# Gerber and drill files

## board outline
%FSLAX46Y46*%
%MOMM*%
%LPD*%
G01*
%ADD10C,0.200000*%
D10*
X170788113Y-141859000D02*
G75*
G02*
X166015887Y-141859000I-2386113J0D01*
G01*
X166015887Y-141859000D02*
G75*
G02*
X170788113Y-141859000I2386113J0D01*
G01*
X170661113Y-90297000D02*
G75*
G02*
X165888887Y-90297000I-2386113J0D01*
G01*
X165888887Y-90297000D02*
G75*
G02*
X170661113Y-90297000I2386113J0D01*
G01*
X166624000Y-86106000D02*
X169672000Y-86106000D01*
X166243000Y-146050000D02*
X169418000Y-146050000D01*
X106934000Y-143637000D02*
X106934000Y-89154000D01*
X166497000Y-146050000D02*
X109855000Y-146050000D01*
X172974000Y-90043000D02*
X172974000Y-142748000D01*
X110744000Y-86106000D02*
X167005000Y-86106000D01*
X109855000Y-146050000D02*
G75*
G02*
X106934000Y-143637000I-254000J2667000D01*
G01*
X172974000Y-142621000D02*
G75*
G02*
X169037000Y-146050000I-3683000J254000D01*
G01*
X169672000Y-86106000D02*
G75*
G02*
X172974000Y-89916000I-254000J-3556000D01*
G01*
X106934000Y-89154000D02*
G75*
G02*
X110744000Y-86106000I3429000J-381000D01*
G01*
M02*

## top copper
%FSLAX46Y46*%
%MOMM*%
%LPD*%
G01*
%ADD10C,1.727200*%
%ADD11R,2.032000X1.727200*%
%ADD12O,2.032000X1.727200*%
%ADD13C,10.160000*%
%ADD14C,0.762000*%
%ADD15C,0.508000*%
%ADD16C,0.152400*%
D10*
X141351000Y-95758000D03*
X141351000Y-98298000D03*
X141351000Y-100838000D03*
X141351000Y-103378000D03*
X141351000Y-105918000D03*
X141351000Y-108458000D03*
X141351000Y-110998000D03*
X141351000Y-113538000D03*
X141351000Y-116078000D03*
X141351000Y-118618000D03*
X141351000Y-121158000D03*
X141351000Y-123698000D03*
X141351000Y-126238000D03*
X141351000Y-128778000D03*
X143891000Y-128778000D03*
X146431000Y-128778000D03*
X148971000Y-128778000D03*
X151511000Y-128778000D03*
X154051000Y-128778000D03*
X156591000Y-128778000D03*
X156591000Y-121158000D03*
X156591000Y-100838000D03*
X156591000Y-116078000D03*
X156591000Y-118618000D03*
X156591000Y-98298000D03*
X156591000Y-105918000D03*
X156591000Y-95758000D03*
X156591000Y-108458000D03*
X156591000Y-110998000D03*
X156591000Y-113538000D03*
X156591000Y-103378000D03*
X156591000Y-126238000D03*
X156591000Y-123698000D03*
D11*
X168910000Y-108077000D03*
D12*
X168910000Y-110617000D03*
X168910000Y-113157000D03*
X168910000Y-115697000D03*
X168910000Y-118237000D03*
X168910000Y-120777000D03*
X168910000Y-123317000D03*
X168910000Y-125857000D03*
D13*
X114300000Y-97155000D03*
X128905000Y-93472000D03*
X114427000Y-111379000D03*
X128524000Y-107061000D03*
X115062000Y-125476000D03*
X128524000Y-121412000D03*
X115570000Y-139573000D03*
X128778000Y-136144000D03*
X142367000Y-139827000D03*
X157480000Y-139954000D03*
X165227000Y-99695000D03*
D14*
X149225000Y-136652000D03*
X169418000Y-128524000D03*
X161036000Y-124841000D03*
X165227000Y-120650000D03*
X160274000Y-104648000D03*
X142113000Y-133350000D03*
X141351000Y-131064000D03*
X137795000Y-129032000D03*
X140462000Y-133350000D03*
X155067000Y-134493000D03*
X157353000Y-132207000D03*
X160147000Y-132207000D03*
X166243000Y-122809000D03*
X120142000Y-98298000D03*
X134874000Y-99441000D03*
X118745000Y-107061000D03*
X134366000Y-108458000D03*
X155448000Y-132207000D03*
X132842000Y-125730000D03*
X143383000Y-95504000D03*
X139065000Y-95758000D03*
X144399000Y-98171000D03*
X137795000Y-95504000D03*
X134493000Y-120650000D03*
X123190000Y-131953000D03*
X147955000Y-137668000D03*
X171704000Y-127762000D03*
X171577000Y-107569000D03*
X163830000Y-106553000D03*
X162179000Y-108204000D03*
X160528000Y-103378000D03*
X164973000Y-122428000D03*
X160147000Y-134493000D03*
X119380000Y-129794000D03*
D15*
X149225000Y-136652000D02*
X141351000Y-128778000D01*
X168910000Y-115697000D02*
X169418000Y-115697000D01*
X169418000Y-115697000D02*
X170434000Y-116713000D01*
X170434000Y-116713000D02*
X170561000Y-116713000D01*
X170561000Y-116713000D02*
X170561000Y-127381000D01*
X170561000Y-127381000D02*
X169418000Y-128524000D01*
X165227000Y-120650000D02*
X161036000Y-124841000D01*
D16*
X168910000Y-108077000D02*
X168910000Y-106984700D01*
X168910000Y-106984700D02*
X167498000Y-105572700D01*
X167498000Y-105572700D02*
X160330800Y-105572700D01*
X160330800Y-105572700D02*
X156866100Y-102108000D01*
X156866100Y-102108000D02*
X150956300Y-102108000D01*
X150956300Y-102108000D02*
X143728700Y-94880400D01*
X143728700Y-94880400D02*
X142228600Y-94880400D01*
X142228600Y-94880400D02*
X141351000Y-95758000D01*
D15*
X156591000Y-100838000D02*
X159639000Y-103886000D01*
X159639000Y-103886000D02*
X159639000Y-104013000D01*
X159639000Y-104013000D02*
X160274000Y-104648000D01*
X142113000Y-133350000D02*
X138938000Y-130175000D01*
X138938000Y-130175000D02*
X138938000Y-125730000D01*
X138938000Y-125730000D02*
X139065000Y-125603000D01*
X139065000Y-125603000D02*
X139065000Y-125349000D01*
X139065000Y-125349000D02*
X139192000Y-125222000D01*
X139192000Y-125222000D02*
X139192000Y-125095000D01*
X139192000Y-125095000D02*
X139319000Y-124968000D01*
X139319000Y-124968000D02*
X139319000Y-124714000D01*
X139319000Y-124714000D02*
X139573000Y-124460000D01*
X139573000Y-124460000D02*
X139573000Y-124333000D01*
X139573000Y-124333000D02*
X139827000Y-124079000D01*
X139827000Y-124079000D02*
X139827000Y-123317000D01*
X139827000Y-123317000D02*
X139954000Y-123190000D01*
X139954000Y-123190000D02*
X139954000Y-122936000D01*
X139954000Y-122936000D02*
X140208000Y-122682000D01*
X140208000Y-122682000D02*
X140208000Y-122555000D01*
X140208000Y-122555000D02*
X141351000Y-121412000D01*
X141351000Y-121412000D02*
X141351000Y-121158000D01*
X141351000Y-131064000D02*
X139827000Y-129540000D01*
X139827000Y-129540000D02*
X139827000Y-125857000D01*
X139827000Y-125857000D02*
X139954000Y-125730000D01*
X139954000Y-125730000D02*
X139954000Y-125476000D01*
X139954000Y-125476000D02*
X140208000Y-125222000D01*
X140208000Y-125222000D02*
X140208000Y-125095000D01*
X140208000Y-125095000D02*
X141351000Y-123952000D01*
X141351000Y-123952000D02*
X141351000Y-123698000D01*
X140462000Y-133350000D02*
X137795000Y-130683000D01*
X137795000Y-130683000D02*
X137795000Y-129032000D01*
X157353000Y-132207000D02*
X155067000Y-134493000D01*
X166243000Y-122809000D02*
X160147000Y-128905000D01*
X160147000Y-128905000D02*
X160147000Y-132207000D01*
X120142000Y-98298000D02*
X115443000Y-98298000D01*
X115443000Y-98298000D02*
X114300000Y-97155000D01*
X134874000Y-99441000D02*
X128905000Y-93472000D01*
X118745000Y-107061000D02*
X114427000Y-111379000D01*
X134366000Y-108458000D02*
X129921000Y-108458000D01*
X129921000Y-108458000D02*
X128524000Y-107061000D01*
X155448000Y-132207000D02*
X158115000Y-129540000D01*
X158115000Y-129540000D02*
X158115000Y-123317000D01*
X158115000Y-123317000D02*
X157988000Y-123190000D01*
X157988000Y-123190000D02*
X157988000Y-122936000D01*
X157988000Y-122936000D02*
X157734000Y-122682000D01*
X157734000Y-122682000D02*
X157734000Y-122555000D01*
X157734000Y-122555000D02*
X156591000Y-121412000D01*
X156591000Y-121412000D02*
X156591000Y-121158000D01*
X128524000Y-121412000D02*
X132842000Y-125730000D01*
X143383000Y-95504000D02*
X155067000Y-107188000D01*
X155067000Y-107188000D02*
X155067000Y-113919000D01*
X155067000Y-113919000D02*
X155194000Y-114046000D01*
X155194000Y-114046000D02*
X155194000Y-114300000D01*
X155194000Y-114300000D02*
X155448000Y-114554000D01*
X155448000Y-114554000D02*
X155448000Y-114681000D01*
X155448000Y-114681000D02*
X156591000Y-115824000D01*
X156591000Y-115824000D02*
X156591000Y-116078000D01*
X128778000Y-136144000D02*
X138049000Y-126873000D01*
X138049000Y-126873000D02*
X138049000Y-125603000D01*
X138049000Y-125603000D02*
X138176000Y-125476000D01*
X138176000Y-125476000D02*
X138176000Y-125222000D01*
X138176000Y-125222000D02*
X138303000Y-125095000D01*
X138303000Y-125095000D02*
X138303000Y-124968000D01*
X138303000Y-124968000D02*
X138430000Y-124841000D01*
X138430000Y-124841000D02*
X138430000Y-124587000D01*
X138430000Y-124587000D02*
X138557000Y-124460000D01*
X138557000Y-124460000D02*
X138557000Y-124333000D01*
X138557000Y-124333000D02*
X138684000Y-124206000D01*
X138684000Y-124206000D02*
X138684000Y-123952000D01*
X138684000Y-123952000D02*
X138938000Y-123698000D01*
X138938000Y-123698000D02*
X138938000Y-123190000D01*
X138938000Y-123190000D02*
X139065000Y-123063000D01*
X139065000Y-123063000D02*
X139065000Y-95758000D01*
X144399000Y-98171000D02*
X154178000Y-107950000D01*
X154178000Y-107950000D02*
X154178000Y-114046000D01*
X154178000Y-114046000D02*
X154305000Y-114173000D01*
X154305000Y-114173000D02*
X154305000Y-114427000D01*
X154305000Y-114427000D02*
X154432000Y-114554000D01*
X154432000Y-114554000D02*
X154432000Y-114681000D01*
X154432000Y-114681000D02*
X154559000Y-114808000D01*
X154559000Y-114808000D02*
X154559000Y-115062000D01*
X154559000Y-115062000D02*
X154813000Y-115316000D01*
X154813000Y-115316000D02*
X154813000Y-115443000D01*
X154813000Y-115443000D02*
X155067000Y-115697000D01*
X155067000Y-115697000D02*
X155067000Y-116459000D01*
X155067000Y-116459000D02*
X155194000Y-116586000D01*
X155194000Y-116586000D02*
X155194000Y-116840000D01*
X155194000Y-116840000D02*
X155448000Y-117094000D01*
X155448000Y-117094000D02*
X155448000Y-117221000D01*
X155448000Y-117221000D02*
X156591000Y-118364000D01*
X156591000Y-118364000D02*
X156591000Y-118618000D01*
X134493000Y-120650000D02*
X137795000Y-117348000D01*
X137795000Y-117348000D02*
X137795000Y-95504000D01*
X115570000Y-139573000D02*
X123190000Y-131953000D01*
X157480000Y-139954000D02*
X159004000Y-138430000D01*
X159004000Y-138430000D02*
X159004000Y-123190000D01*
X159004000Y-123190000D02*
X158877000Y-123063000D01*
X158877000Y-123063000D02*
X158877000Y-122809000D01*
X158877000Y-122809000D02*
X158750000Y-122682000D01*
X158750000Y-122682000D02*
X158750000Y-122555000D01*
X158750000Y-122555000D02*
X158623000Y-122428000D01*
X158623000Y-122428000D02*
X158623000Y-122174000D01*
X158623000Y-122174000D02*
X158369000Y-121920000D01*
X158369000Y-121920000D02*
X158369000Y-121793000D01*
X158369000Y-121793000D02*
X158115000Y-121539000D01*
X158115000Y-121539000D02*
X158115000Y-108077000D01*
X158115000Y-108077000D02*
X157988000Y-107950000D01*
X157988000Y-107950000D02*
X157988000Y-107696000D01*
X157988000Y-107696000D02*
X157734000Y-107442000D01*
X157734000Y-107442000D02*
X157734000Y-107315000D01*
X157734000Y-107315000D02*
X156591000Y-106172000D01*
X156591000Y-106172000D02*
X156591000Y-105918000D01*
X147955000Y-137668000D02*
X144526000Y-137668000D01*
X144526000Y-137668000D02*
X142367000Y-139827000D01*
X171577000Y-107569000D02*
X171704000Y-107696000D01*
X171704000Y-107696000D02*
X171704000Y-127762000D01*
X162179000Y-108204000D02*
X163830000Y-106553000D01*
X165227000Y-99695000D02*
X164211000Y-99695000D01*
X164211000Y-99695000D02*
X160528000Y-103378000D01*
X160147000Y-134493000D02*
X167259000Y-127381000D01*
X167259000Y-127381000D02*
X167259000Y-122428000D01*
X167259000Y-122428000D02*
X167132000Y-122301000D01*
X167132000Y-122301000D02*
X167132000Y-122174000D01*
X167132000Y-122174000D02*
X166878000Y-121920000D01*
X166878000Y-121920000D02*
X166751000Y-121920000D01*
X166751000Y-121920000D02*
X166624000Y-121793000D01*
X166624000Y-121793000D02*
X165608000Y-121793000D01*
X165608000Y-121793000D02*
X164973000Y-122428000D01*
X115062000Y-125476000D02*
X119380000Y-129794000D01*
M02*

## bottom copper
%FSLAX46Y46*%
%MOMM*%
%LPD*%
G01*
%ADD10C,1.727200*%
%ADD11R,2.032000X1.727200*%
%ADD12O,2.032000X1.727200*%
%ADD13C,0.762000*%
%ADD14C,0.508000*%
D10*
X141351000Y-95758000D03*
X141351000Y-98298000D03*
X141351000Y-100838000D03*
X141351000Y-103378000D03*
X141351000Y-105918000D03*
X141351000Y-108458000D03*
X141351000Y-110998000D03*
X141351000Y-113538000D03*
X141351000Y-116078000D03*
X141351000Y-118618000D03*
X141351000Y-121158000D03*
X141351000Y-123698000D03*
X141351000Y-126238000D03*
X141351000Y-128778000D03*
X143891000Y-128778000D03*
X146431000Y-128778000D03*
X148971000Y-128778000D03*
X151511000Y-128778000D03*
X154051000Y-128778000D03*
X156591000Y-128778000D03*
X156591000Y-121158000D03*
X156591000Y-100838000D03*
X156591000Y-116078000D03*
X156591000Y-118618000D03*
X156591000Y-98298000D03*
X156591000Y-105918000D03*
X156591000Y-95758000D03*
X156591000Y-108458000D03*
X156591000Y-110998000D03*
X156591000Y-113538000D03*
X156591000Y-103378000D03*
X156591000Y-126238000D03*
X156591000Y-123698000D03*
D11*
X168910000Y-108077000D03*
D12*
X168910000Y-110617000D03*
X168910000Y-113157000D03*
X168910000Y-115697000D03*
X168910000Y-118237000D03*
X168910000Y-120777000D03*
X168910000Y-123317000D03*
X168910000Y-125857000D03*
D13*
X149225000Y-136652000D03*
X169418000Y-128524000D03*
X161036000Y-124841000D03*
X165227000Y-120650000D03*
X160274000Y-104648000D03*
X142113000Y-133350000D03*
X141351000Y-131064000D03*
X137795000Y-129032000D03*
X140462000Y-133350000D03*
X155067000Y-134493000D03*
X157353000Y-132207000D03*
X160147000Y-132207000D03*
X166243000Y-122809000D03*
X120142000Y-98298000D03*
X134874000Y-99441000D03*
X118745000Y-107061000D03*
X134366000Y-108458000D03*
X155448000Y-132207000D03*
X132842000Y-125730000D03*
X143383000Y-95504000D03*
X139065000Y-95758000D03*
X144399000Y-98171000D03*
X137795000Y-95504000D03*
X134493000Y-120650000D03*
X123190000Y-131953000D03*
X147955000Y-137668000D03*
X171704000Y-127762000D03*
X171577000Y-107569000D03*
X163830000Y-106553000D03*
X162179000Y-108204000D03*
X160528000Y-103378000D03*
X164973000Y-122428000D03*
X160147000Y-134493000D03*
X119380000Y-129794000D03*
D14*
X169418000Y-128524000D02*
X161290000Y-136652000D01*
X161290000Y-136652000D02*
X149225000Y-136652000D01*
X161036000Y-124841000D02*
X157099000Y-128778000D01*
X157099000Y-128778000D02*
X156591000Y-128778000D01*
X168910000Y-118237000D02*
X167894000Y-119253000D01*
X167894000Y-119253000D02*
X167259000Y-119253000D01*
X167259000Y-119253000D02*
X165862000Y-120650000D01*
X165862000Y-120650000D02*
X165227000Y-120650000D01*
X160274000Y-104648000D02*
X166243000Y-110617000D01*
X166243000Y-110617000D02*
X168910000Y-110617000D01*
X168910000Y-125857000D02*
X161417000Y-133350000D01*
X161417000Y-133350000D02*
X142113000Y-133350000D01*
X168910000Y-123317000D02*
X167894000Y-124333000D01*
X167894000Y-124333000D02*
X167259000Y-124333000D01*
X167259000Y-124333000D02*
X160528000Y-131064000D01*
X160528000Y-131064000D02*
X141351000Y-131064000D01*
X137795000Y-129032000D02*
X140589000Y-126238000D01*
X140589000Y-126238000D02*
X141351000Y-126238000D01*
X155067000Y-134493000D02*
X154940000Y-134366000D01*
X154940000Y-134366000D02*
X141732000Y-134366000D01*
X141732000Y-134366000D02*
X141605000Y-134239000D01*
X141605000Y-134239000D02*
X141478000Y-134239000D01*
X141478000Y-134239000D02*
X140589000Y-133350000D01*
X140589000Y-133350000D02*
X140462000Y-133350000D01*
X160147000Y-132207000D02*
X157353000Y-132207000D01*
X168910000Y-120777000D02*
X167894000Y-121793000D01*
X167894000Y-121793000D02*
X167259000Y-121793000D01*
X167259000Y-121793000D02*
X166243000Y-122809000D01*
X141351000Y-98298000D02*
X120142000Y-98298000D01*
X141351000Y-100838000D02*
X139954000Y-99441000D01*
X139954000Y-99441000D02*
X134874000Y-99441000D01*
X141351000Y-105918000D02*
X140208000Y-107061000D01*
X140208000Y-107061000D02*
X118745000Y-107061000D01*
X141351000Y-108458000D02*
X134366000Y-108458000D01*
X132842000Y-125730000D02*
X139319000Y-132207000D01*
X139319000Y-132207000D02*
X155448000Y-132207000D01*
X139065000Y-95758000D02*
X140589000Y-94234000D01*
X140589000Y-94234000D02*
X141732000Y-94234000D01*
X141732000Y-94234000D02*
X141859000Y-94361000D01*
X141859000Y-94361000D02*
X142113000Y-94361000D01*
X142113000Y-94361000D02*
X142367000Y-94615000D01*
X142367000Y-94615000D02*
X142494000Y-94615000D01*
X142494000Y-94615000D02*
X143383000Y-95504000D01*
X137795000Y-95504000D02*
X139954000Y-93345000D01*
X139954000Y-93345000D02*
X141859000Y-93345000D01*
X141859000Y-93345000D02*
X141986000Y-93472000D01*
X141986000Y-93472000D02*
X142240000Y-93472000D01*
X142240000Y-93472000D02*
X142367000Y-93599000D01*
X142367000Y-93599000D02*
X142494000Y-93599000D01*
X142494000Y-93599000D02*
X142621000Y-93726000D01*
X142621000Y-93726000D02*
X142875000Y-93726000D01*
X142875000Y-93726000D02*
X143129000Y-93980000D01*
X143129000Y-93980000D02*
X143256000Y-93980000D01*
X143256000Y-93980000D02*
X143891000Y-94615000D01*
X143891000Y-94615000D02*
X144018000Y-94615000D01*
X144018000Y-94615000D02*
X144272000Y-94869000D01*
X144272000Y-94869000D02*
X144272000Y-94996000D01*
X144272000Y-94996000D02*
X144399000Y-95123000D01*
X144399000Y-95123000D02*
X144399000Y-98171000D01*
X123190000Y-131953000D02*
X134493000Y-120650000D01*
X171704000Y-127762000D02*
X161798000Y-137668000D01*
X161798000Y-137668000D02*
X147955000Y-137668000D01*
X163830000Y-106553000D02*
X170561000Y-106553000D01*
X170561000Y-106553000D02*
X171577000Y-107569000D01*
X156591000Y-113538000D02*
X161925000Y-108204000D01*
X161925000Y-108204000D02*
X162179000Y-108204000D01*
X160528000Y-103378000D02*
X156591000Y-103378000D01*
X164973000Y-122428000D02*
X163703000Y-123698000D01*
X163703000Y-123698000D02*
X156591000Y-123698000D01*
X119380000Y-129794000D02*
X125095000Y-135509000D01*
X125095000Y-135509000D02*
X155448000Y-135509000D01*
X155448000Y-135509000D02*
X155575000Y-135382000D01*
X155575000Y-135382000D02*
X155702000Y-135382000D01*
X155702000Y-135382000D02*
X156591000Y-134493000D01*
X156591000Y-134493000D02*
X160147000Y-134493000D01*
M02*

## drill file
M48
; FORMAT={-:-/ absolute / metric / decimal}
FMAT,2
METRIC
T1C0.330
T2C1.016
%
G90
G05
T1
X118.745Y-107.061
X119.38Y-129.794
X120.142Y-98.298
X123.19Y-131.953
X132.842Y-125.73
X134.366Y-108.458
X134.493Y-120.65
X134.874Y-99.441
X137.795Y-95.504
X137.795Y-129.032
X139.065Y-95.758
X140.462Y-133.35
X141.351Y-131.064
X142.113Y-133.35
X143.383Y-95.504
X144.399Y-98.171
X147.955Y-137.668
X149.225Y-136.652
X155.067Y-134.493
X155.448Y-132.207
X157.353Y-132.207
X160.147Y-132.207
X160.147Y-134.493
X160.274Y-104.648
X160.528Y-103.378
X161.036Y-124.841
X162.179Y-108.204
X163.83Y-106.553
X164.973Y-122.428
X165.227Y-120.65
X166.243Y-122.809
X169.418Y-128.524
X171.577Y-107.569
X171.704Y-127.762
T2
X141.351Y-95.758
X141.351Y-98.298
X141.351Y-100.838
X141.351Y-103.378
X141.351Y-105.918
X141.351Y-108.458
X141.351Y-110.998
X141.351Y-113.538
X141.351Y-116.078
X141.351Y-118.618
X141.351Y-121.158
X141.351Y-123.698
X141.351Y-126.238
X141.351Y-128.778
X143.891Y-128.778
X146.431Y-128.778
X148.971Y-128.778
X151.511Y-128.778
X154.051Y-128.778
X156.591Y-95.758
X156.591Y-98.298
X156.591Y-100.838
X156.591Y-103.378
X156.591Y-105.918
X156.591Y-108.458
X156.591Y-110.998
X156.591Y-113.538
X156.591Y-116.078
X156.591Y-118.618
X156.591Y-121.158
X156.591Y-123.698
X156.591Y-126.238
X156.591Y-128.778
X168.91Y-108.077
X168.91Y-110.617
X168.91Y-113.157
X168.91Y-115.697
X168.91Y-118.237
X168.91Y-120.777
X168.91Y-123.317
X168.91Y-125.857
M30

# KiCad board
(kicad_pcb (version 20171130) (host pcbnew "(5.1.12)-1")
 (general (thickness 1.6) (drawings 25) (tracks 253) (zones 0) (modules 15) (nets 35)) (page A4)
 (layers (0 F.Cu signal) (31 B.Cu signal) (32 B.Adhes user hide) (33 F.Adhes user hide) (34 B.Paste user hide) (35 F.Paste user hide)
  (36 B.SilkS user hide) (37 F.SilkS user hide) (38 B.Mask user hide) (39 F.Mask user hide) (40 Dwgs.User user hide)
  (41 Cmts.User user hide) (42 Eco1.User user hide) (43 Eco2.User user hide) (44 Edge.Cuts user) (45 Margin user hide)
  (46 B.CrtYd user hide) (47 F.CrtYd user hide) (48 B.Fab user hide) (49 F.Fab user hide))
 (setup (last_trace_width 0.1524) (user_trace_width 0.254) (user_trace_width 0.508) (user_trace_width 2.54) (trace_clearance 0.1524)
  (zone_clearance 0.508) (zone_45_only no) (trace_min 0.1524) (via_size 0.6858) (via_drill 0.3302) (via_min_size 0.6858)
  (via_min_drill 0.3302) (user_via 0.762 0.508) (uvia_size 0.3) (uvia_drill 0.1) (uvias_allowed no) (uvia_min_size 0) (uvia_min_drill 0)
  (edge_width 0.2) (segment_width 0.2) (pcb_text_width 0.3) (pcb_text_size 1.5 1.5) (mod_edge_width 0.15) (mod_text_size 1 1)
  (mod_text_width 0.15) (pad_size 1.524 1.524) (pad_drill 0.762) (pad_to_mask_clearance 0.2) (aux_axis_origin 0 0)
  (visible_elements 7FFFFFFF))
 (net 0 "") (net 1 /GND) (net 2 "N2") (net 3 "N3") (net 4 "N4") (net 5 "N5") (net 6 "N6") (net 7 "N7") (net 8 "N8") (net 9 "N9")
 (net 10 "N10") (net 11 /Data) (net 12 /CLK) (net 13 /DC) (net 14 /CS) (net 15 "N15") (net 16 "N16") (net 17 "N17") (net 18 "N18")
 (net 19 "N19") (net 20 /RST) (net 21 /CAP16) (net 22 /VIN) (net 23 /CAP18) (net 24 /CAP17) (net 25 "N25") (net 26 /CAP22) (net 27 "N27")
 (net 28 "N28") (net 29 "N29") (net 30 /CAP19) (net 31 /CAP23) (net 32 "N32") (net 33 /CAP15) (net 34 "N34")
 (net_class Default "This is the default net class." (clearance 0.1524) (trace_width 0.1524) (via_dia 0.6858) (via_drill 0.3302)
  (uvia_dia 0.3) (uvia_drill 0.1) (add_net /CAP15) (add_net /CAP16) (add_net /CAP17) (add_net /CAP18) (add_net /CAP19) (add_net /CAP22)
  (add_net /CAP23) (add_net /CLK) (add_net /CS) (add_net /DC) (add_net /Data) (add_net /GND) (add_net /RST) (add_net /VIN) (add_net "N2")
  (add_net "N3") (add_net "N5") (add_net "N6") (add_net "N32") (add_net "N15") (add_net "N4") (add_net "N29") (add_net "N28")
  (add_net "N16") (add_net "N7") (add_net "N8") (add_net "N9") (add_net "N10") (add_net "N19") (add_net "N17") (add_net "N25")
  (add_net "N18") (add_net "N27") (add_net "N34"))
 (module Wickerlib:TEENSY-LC (layer F.Cu) (at 151.511 105.918)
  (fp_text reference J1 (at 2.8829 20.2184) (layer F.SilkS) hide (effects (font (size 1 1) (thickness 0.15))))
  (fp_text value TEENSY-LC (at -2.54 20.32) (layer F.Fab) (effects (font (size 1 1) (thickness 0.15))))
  (pad G1 thru_hole circle (at -10.16 -10.16) (size 1.7272 1.7272) (drill 1.016) (layers *.Cu *.Mask F.SilkS) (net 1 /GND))
  (pad 0 thru_hole circle (at -10.16 -7.62) (size 1.7272 1.7272) (drill 1.016) (layers *.Cu *.Mask F.SilkS) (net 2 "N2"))
  (pad 1 thru_hole circle (at -10.16 -5.08) (size 1.7272 1.7272) (drill 1.016) (layers *.Cu *.Mask F.SilkS) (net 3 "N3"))
  (pad 2 thru_hole circle (at -10.16 -2.54) (size 1.7272 1.7272) (drill 1.016) (layers *.Cu *.Mask F.SilkS) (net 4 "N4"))
  (pad 3 thru_hole circle (at -10.16 0) (size 1.7272 1.7272) (drill 1.016) (layers *.Cu *.Mask F.SilkS) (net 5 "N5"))
  (pad 4 thru_hole circle (at -10.16 2.54) (size 1.7272 1.7272) (drill 1.016) (layers *.Cu *.Mask F.SilkS) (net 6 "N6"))
  (pad 5 thru_hole circle (at -10.16 5.08) (size 1.7272 1.7272) (drill 1.016) (layers *.Cu *.Mask F.SilkS) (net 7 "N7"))
  (pad 6 thru_hole circle (at -10.16 7.62) (size 1.7272 1.7272) (drill 1.016) (layers *.Cu *.Mask F.SilkS) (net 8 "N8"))
  (pad 7 thru_hole circle (at -10.16 10.16) (size 1.7272 1.7272) (drill 1.016) (layers *.Cu *.Mask F.SilkS) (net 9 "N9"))
  (pad 8 thru_hole circle (at -10.16 12.7) (size 1.7272 1.7272) (drill 1.016) (layers *.Cu *.Mask F.SilkS) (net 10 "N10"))
  (pad 9 thru_hole circle (at -10.16 15.24) (size 1.7272 1.7272) (drill 1.016) (layers *.Cu *.Mask F.SilkS) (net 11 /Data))
  (pad 10 thru_hole circle (at -10.16 17.78) (size 1.7272 1.7272) (drill 1.016) (layers *.Cu *.Mask F.SilkS) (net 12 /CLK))
  (pad 11 thru_hole circle (at -10.16 20.32) (size 1.7272 1.7272) (drill 1.016) (layers *.Cu *.Mask F.SilkS) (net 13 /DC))
  (pad 12 thru_hole circle (at -10.16 22.86) (size 1.7272 1.7272) (drill 1.016) (layers *.Cu *.Mask F.SilkS) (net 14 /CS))
  (pad 17A thru_hole circle (at -7.62 22.86) (size 1.7272 1.7272) (drill 1.016) (layers *.Cu *.Mask F.SilkS) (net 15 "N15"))
  (pad 3V1 thru_hole circle (at -5.08 22.86) (size 1.7272 1.7272) (drill 1.016) (layers *.Cu *.Mask F.SilkS) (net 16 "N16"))
  (pad G2 thru_hole circle (at -2.54 22.86) (size 1.7272 1.7272) (drill 1.016) (layers *.Cu *.Mask F.SilkS) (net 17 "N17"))
  (pad PGM thru_hole circle (at 0 22.86) (size 1.7272 1.7272) (drill 1.016) (layers *.Cu *.Mask F.SilkS) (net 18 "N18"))
  (pad DAC thru_hole circle (at 2.54 22.86) (size 1.7272 1.7272) (drill 1.016) (layers *.Cu *.Mask F.SilkS) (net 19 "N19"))
  (pad 13 thru_hole circle (at 5.08 22.86) (size 1.7272 1.7272) (drill 1.016) (layers *.Cu *.Mask F.SilkS) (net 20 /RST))
  (pad 16 thru_hole circle (at 5.08 15.24) (size 1.7272 1.7272) (drill 1.016) (layers *.Cu *.Mask F.SilkS) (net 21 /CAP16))
  (pad 3V2 thru_hole circle (at 5.08 -5.08) (size 1.7272 1.7272) (drill 1.016) (layers *.Cu *.Mask F.SilkS) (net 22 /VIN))
  (pad 18 thru_hole circle (at 5.08 10.16) (size 1.7272 1.7272) (drill 1.016) (layers *.Cu *.Mask F.SilkS) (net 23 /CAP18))
  (pad 17 thru_hole circle (at 5.08 12.7) (size 1.7272 1.7272) (drill 1.016) (layers *.Cu *.Mask F.SilkS) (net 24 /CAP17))
  (pad G3 thru_hole circle (at 5.08 -7.62) (size 1.7272 1.7272) (drill 1.016) (layers *.Cu *.Mask F.SilkS) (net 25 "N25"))
  (pad 22 thru_hole circle (at 5.08 0) (size 1.7272 1.7272) (drill 1.016) (layers *.Cu *.Mask F.SilkS) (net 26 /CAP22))
  (pad VIN thru_hole circle (at 5.08 -10.16) (size 1.7272 1.7272) (drill 1.016) (layers *.Cu *.Mask F.SilkS) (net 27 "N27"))
  (pad 21 thru_hole circle (at 5.08 2.54) (size 1.7272 1.7272) (drill 1.016) (layers *.Cu *.Mask F.SilkS) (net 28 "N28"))
  (pad 20 thru_hole circle (at 5.08 5.08) (size 1.7272 1.7272) (drill 1.016) (layers *.Cu *.Mask F.SilkS) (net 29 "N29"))
  (pad 19 thru_hole circle (at 5.08 7.62) (size 1.7272 1.7272) (drill 1.016) (layers *.Cu *.Mask F.SilkS) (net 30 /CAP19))
  (pad 23 thru_hole circle (at 5.08 -2.54) (size 1.7272 1.7272) (drill 1.016) (layers *.Cu *.Mask F.SilkS) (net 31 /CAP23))
  (pad 14 thru_hole circle (at 5.08 20.32) (size 1.7272 1.7272) (drill 1.016) (layers *.Cu *.Mask F.SilkS) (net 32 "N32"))
  (pad 15 thru_hole circle (at 5.08 17.78) (size 1.7272 1.7272) (drill 1.016) (layers *.Cu *.Mask F.SilkS) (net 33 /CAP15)))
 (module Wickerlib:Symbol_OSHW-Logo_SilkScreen (layer F.Cu) (at 167.767 133.985 270)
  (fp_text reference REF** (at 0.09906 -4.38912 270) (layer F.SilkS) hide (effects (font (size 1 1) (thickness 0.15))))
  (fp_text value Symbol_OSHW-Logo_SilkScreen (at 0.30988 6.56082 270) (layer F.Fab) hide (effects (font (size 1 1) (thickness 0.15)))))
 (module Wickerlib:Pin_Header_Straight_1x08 (layer F.Cu) (at 168.91 108.077)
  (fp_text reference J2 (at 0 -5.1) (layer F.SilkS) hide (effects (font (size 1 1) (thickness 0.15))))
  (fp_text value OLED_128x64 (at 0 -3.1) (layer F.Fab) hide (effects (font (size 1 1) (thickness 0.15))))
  (pad 1 thru_hole rect (at 0 0) (size 2.032 1.7272) (drill 1.016) (layers *.Cu *.Mask F.SilkS) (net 1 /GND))
  (pad 2 thru_hole oval (at 0 2.54) (size 2.032 1.7272) (drill 1.016) (layers *.Cu *.Mask F.SilkS) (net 22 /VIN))
  (pad 3 thru_hole oval (at 0 5.08) (size 2.032 1.7272) (drill 1.016) (layers *.Cu *.Mask F.SilkS) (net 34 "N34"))
  (pad 4 thru_hole oval (at 0 7.62) (size 2.032 1.7272) (drill 1.016) (layers *.Cu *.Mask F.SilkS) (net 14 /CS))
  (pad 5 thru_hole oval (at 0 10.16) (size 2.032 1.7272) (drill 1.016) (layers *.Cu *.Mask F.SilkS) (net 20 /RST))
  (pad 6 thru_hole oval (at 0 12.7) (size 2.032 1.7272) (drill 1.016) (layers *.Cu *.Mask F.SilkS) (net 13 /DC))
  (pad 7 thru_hole oval (at 0 15.24) (size 2.032 1.7272) (drill 1.016) (layers *.Cu *.Mask F.SilkS) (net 12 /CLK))
  (pad 8 thru_hole oval (at 0 17.78) (size 2.032 1.7272) (drill 1.016) (layers *.Cu *.Mask F.SilkS) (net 11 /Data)))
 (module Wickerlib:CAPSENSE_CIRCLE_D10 (layer F.Cu) (at 114.3 97.155)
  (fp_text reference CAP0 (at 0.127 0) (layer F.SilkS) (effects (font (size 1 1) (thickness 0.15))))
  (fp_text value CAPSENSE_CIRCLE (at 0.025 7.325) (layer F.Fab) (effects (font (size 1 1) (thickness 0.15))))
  (pad 1 smd circle (at 0 0) (size 10.16 10.16) (layers F.Cu) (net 2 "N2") (clearance 0.508)))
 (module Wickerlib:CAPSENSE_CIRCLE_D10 (layer F.Cu) (at 128.905 93.472 90)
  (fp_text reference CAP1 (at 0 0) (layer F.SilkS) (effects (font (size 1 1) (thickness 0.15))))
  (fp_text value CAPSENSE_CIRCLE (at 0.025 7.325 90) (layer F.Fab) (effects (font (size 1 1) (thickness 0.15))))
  (pad 1 smd circle (at 0 0 90) (size 10.16 10.16) (layers F.Cu) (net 3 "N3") (clearance 0.508)))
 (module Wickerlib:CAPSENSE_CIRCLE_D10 (layer F.Cu) (at 114.427 111.379)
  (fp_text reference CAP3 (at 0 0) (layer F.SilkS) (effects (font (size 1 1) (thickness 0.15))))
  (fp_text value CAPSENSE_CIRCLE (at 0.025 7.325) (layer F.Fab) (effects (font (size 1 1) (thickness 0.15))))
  (pad 1 smd circle (at 0 0) (size 10.16 10.16) (layers F.Cu) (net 5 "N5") (clearance 0.508)))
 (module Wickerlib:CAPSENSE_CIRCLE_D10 (layer F.Cu) (at 128.524 107.061)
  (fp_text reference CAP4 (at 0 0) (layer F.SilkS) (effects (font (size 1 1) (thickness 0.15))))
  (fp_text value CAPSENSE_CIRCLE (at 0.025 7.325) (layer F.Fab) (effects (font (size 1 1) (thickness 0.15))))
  (pad 1 smd circle (at 0 0) (size 10.16 10.16) (layers F.Cu) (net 6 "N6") (clearance 0.508)))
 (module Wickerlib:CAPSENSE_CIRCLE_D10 (layer F.Cu) (at 115.062 125.476)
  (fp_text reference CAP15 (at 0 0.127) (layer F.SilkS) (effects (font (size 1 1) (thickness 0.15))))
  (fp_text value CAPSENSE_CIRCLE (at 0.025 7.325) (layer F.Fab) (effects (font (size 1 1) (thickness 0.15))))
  (pad 1 smd circle (at 0 0) (size 10.16 10.16) (layers F.Cu) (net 33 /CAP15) (clearance 0.508)))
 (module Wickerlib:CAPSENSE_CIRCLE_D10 (layer F.Cu) (at 128.524 121.412)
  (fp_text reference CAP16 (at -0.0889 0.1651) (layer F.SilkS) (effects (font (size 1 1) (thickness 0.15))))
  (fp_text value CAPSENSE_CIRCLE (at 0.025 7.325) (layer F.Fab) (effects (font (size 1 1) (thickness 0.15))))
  (pad 1 smd circle (at 0 0) (size 10.16 10.16) (layers F.Cu) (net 21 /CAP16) (clearance 0.508)))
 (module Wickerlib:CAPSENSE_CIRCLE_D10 (layer F.Cu) (at 115.57 139.573)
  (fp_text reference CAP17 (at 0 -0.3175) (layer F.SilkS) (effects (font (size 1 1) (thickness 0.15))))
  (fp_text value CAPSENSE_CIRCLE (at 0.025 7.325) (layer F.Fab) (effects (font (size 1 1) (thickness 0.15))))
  (pad 1 smd circle (at 0 0) (size 10.16 10.16) (layers F.Cu) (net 24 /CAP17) (clearance 0.508)))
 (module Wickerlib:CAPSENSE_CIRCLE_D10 (layer F.Cu) (at 128.778 136.144)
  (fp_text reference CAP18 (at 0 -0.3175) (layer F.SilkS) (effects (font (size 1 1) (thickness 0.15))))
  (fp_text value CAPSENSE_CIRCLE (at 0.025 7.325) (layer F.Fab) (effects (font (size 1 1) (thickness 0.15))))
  (pad 1 smd circle (at 0 0) (size 10.16 10.16) (layers F.Cu) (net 23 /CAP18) (clearance 0.508)))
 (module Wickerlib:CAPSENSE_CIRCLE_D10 (layer F.Cu) (at 142.367 139.827)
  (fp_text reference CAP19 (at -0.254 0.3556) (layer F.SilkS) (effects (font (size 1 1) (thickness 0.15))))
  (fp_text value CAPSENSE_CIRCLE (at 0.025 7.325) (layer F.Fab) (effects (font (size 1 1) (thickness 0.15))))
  (pad 1 smd circle (at 0 0) (size 10.16 10.16) (layers F.Cu) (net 30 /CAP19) (clearance 0.508)))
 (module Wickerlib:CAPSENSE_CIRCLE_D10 (layer F.Cu) (at 157.48 139.954)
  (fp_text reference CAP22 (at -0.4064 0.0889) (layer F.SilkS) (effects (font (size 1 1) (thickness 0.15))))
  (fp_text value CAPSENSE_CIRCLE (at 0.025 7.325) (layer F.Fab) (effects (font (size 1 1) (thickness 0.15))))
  (pad 1 smd circle (at 0 0) (size 10.16 10.16) (layers F.Cu) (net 26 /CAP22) (clearance 0.508)))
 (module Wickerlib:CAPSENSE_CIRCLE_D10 (layer F.Cu) (at 165.227 99.695)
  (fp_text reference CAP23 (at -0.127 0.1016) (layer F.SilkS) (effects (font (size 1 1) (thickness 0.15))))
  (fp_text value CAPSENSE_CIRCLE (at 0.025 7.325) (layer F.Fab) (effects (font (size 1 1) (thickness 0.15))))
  (pad 1 smd circle (at 0 0) (size 10.16 10.16) (layers F.Cu) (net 31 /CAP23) (clearance 0.508)))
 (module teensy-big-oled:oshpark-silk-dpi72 (layer B.Cu) (at 140.843 116.967)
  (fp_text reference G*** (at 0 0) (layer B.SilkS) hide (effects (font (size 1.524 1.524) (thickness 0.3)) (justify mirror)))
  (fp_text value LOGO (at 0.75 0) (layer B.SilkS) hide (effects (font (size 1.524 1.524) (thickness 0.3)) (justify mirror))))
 (gr_circle (center 168.402 141.859) (end 167.386 139.7) (layer Edge.Cuts) (width 0.2))
 (gr_circle (center 168.275 90.297) (end 167.259 88.138) (layer Edge.Cuts) (width 0.2))
 (gr_line (start 166.624 86.106) (end 169.672 86.106) (angle 90) (layer Edge.Cuts) (width 0.2))
 (gr_line (start 166.243 146.05) (end 169.418 146.05) (angle 90) (layer Edge.Cuts) (width 0.2))
 (gr_line (start 106.934 143.637) (end 106.934 89.154) (angle 90) (layer Edge.Cuts) (width 0.2))
 (gr_line (start 166.497 146.05) (end 109.855 146.05) (angle 90) (layer Edge.Cuts) (width 0.2))
 (gr_line (start 172.974 90.043) (end 172.974 142.748) (angle 90) (layer Edge.Cuts) (width 0.2))
 (gr_line (start 110.744 86.106) (end 167.005 86.106) (angle 90) (layer Edge.Cuts) (width 0.2))
 (gr_arc (start 109.601 143.383) (end 109.855 146.05) (angle 90) (layer Edge.Cuts) (width 0.2))
 (gr_arc (start 169.291 142.367) (end 172.974 142.621) (angle 90) (layer Edge.Cuts) (width 0.2))
 (gr_arc (start 169.418 89.662) (end 169.672 86.106) (angle 90) (layer Edge.Cuts) (width 0.2))
 (gr_arc (start 110.363 89.535) (end 106.934 89.154) (angle 90) (layer Edge.Cuts) (width 0.2))
 (segment (start 149.225 136.652) (end 141.351 128.778) (width 0.508) (layer F.Cu) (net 14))
 (segment (start 169.418 128.524) (end 161.29 136.652) (width 0.508) (layer B.Cu) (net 14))
 (segment (start 161.29 136.652) (end 149.225 136.652) (width 0.508) (layer B.Cu) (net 14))
 (segment (start 168.91 115.697) (end 169.418 115.697) (width 0.508) (layer F.Cu) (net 14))
 (segment (start 169.418 115.697) (end 170.434 116.713) (width 0.508) (layer F.Cu) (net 14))
 (segment (start 170.434 116.713) (end 170.561 116.713) (width 0.508) (layer F.Cu) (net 14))
 (segment (start 170.561 116.713) (end 170.561 127.381) (width 0.508) (layer F.Cu) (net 14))
 (segment (start 170.561 127.381) (end 169.418 128.524) (width 0.508) (layer F.Cu) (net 14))
 (via (at 149.225 136.652) (size 0.762) (layers F.Cu B.Cu) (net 14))
 (via (at 169.418 128.524) (size 0.762) (layers F.Cu B.Cu) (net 14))
 (segment (start 161.036 124.841) (end 157.099 128.778) (width 0.508) (layer B.Cu) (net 20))
 (segment (start 157.099 128.778) (end 156.591 128.778) (width 0.508) (layer B.Cu) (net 20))
 (segment (start 165.227 120.65) (end 161.036 124.841) (width 0.508) (layer F.Cu) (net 20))
 (segment (start 168.91 118.237) (end 167.894 119.253) (width 0.508) (layer B.Cu) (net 20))
 (segment (start 167.894 119.253) (end 167.259 119.253) (width 0.508) (layer B.Cu) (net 20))
 (segment (start 167.259 119.253) (end 165.862 120.65) (width 0.508) (layer B.Cu) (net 20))
 (segment (start 165.862 120.65) (end 165.227 120.65) (width 0.508) (layer B.Cu) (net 20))
 (via (at 161.036 124.841) (size 0.762) (layers F.Cu B.Cu) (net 20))
 (via (at 165.227 120.65) (size 0.762) (layers F.Cu B.Cu) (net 20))
 (segment (start 168.91 108.077) (end 168.91 106.9847) (width 0.1524) (layer F.Cu) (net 1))
 (segment (start 168.91 106.9847) (end 167.498 105.5727) (width 0.1524) (layer F.Cu) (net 1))
 (segment (start 167.498 105.5727) (end 160.3308 105.5727) (width 0.1524) (layer F.Cu) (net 1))
 (segment (start 160.3308 105.5727) (end 156.8661 102.108) (width 0.1524) (layer F.Cu) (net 1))
 (segment (start 156.8661 102.108) (end 150.9563 102.108) (width 0.1524) (layer F.Cu) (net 1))
 (segment (start 150.9563 102.108) (end 143.7287 94.8804) (width 0.1524) (layer F.Cu) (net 1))
 (segment (start 143.7287 94.8804) (end 142.2286 94.8804) (width 0.1524) (layer F.Cu) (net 1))
 (segment (start 142.2286 94.8804) (end 141.351 95.758) (width 0.1524) (layer F.Cu) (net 1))
 (segment (start 160.274 104.648) (end 166.243 110.617) (width 0.508) (layer B.Cu) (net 22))
 (segment (start 166.243 110.617) (end 168.91 110.617) (width 0.508) (layer B.Cu) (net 22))
 (segment (start 156.591 100.838) (end 159.639 103.886) (width 0.508) (layer F.Cu) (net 22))
 (segment (start 159.639 103.886) (end 159.639 104.013) (width 0.508) (layer F.Cu) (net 22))
 (segment (start 159.639 104.013) (end 160.274 104.648) (width 0.508) (layer F.Cu) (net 22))
 (via (at 160.274 104.648) (size 0.762) (layers F.Cu B.Cu) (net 22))
 (segment (start 142.113 133.35) (end 138.938 130.175) (width 0.508) (layer F.Cu) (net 11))
 (segment (start 138.938 130.175) (end 138.938 125.73) (width 0.508) (layer F.Cu) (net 11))
 (segment (start 138.938 125.73) (end 139.065 125.603) (width 0.508) (layer F.Cu) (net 11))
 (segment (start 139.065 125.603) (end 139.065 125.349) (width 0.508) (layer F.Cu) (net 11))
 (segment (start 139.065 125.349) (end 139.192 125.222) (width 0.508) (layer F.Cu) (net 11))
 (segment (start 139.192 125.222) (end 139.192 125.095) (width 0.508) (layer F.Cu) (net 11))
 (segment (start 139.192 125.095) (end 139.319 124.968) (width 0.508) (layer F.Cu) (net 11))
 (segment (start 139.319 124.968) (end 139.319 124.714) (width 0.508) (layer F.Cu) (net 11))
 (segment (start 139.319 124.714) (end 139.573 124.46) (width 0.508) (layer F.Cu) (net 11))
 (segment (start 139.573 124.46) (end 139.573 124.333) (width 0.508) (layer F.Cu) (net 11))
 (segment (start 139.573 124.333) (end 139.827 124.079) (width 0.508) (layer F.Cu) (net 11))
 (segment (start 139.827 124.079) (end 139.827 123.317) (width 0.508) (layer F.Cu) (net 11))
 (segment (start 139.827 123.317) (end 139.954 123.19) (width 0.508) (layer F.Cu) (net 11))
 (segment (start 139.954 123.19) (end 139.954 122.936) (width 0.508) (layer F.Cu) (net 11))
 (segment (start 139.954 122.936) (end 140.208 122.682) (width 0.508) (layer F.Cu) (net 11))
 (segment (start 140.208 122.682) (end 140.208 122.555) (width 0.508) (layer F.Cu) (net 11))
 (segment (start 140.208 122.555) (end 141.351 121.412) (width 0.508) (layer F.Cu) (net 11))
 (segment (start 141.351 121.412) (end 141.351 121.158) (width 0.508) (layer F.Cu) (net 11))
 (segment (start 168.91 125.857) (end 161.417 133.35) (width 0.508) (layer B.Cu) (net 11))
 (segment (start 161.417 133.35) (end 142.113 133.35) (width 0.508) (layer B.Cu) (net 11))
 (via (at 142.113 133.35) (size 0.762) (layers F.Cu B.Cu) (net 11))
 (segment (start 141.351 131.064) (end 139.827 129.54) (width 0.508) (layer F.Cu) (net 12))
 (segment (start 139.827 129.54) (end 139.827 125.857) (width 0.508) (layer F.Cu) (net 12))
 (segment (start 139.827 125.857) (end 139.954 125.73) (width 0.508) (layer F.Cu) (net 12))
 (segment (start 139.954 125.73) (end 139.954 125.476) (width 0.508) (layer F.Cu) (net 12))
 (segment (start 139.954 125.476) (end 140.208 125.222) (width 0.508) (layer F.Cu) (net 12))
 (segment (start 140.208 125.222) (end 140.208 125.095) (width 0.508) (layer F.Cu) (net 12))
 (segment (start 140.208 125.095) (end 141.351 123.952) (width 0.508) (layer F.Cu) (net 12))
 (segment (start 141.351 123.952) (end 141.351 123.698) (width 0.508) (layer F.Cu) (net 12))
 (segment (start 168.91 123.317) (end 167.894 124.333) (width 0.508) (layer B.Cu) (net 12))
 (segment (start 167.894 124.333) (end 167.259 124.333) (width 0.508) (layer B.Cu) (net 12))
 (segment (start 167.259 124.333) (end 160.528 131.064) (width 0.508) (layer B.Cu) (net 12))
 (segment (start 160.528 131.064) (end 141.351 131.064) (width 0.508) (layer B.Cu) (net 12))
 (via (at 141.351 131.064) (size 0.762) (layers F.Cu B.Cu) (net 12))
 (segment (start 137.795 129.032) (end 140.589 126.238) (width 0.508) (layer B.Cu) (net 13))
 (segment (start 140.589 126.238) (end 141.351 126.238) (width 0.508) (layer B.Cu) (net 13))
 (segment (start 140.462 133.35) (end 137.795 130.683) (width 0.508) (layer F.Cu) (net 13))
 (segment (start 137.795 130.683) (end 137.795 129.032) (width 0.508) (layer F.Cu) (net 13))
 (segment (start 155.067 134.493) (end 154.94 134.366) (width 0.508) (layer B.Cu) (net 13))
 (segment (start 154.94 134.366) (end 141.732 134.366) (width 0.508) (layer B.Cu) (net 13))
 (segment (start 141.732 134.366) (end 141.605 134.239) (width 0.508) (layer B.Cu) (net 13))
 (segment (start 141.605 134.239) (end 141.478 134.239) (width 0.508) (layer B.Cu) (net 13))
 (segment (start 141.478 134.239) (end 140.589 133.35) (width 0.508) (layer B.Cu) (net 13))
 (segment (start 140.589 133.35) (end 140.462 133.35) (width 0.508) (layer B.Cu) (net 13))
 (segment (start 157.353 132.207) (end 155.067 134.493) (width 0.508) (layer F.Cu) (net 13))
 (segment (start 160.147 132.207) (end 157.353 132.207) (width 0.508) (layer B.Cu) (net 13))
 (segment (start 166.243 122.809) (end 160.147 128.905) (width 0.508) (layer F.Cu) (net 13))
 (segment (start 160.147 128.905) (end 160.147 132.207) (width 0.508) (layer F.Cu) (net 13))
 (segment (start 168.91 120.777) (end 167.894 121.793) (width 0.508) (layer B.Cu) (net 13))
 (segment (start 167.894 121.793) (end 167.259 121.793) (width 0.508) (layer B.Cu) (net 13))
 (segment (start 167.259 121.793) (end 166.243 122.809) (width 0.508) (layer B.Cu) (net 13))
 (via (at 137.795 129.032) (size 0.762) (layers F.Cu B.Cu) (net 13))
 (via (at 140.462 133.35) (size 0.762) (layers F.Cu B.Cu) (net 13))
 (via (at 155.067 134.493) (size 0.762) (layers F.Cu B.Cu) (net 13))
 (via (at 157.353 132.207) (size 0.762) (layers F.Cu B.Cu) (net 13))
 (via (at 160.147 132.207) (size 0.762) (layers F.Cu B.Cu) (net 13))
 (via (at 166.243 122.809) (size 0.762) (layers F.Cu B.Cu) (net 13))
 (segment (start 120.142 98.298) (end 115.443 98.298) (width 0.508) (layer F.Cu) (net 2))
 (segment (start 115.443 98.298) (end 114.3 97.155) (width 0.508) (layer F.Cu) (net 2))
 (segment (start 141.351 98.298) (end 120.142 98.298) (width 0.508) (layer B.Cu) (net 2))
 (via (at 120.142 98.298) (size 0.762) (layers F.Cu B.Cu) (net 2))
 (segment (start 134.874 99.441) (end 128.905 93.472) (width 0.508) (layer F.Cu) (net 3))
 (segment (start 141.351 100.838) (end 139.954 99.441) (width 0.508) (layer B.Cu) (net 3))
 (segment (start 139.954 99.441) (end 134.874 99.441) (width 0.508) (layer B.Cu) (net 3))
 (via (at 134.874 99.441) (size 0.762) (layers F.Cu B.Cu) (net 3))
 (segment (start 118.745 107.061) (end 114.427 111.379) (width 0.508) (layer F.Cu) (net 5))
 (segment (start 141.351 105.918) (end 140.208 107.061) (width 0.508) (layer B.Cu) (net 5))
 (segment (start 140.208 107.061) (end 118.745 107.061) (width 0.508) (layer B.Cu) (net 5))
 (via (at 118.745 107.061) (size 0.762) (layers F.Cu B.Cu) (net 5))
 (segment (start 134.366 108.458) (end 129.921 108.458) (width 0.508) (layer F.Cu) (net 6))
 (segment (start 129.921 108.458) (end 128.524 107.061) (width 0.508) (layer F.Cu) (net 6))
 (segment (start 141.351 108.458) (end 134.366 108.458) (width 0.508) (layer B.Cu) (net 6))
 (via (at 134.366 108.458) (size 0.762) (layers F.Cu B.Cu) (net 6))
 (segment (start 155.448 132.207) (end 158.115 129.54) (width 0.508) (layer F.Cu) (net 21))
 (segment (start 158.115 129.54) (end 158.115 123.317) (width 0.508) (layer F.Cu) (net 21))
 (segment (start 158.115 123.317) (end 157.988 123.19) (width 0.508) (layer F.Cu) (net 21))
 (segment (start 157.988 123.19) (end 157.988 122.936) (width 0.508) (layer F.Cu) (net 21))
 (segment (start 157.988 122.936) (end 157.734 122.682) (width 0.508) (layer F.Cu) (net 21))
 (segment (start 157.734 122.682) (end 157.734 122.555) (width 0.508) (layer F.Cu) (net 21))
 (segment (start 157.734 122.555) (end 156.591 121.412) (width 0.508) (layer F.Cu) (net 21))
 (segment (start 156.591 121.412) (end 156.591 121.158) (width 0.508) (layer F.Cu) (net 21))
 (segment (start 132.842 125.73) (end 139.319 132.207) (width 0.508) (layer B.Cu) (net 21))
 (segment (start 139.319 132.207) (end 155.448 132.207) (width 0.508) (layer B.Cu) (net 21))
 (segment (start 128.524 121.412) (end 132.842 125.73) (width 0.508) (layer F.Cu) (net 21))
 (via (at 155.448 132.207) (size 0.762) (layers F.Cu B.Cu) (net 21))
 (via (at 132.842 125.73) (size 0.762) (layers F.Cu B.Cu) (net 21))
 (segment (start 143.383 95.504) (end 155.067 107.188) (width 0.508) (layer F.Cu) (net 23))
 (segment (start 155.067 107.188) (end 155.067 113.919) (width 0.508) (layer F.Cu) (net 23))
 (segment (start 155.067 113.919) (end 155.194 114.046) (width 0.508) (layer F.Cu) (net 23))
 (segment (start 155.194 114.046) (end 155.194 114.3) (width 0.508) (layer F.Cu) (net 23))
 (segment (start 155.194 114.3) (end 155.448 114.554) (width 0.508) (layer F.Cu) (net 23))
 (segment (start 155.448 114.554) (end 155.448 114.681) (width 0.508) (layer F.Cu) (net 23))
 (segment (start 155.448 114.681) (end 156.591 115.824) (width 0.508) (layer F.Cu) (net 23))
 (segment (start 156.591 115.824) (end 156.591 116.078) (width 0.508) (layer F.Cu) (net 23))
 (segment (start 139.065 95.758) (end 140.589 94.234) (width 0.508) (layer B.Cu) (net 23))
 (segment (start 140.589 94.234) (end 141.732 94.234) (width 0.508) (layer B.Cu) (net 23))
 (segment (start 141.732 94.234) (end 141.859 94.361) (width 0.508) (layer B.Cu) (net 23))
 (segment (start 141.859 94.361) (end 142.113 94.361) (width 0.508) (layer B.Cu) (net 23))
 (segment (start 142.113 94.361) (end 142.367 94.615) (width 0.508) (layer B.Cu) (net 23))
 (segment (start 142.367 94.615) (end 142.494 94.615) (width 0.508) (layer B.Cu) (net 23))
 (segment (start 142.494 94.615) (end 143.383 95.504) (width 0.508) (layer B.Cu) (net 23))
 (segment (start 128.778 136.144) (end 138.049 126.873) (width 0.508) (layer F.Cu) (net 23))
 (segment (start 138.049 126.873) (end 138.049 125.603) (width 0.508) (layer F.Cu) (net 23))
 (segment (start 138.049 125.603) (end 138.176 125.476) (width 0.508) (layer F.Cu) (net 23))
 (segment (start 138.176 125.476) (end 138.176 125.222) (width 0.508) (layer F.Cu) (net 23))
 (segment (start 138.176 125.222) (end 138.303 125.095) (width 0.508) (layer F.Cu) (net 23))
 (segment (start 138.303 125.095) (end 138.303 124.968) (width 0.508) (layer F.Cu) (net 23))
 (segment (start 138.303 124.968) (end 138.43 124.841) (width 0.508) (layer F.Cu) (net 23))
 (segment (start 138.43 124.841) (end 138.43 124.587) (width 0.508) (layer F.Cu) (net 23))
 (segment (start 138.43 124.587) (end 138.557 124.46) (width 0.508) (layer F.Cu) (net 23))
 (segment (start 138.557 124.46) (end 138.557 124.333) (width 0.508) (layer F.Cu) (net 23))
 (segment (start 138.557 124.333) (end 138.684 124.206) (width 0.508) (layer F.Cu) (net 23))
 (segment (start 138.684 124.206) (end 138.684 123.952) (width 0.508) (layer F.Cu) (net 23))
 (segment (start 138.684 123.952) (end 138.938 123.698) (width 0.508) (layer F.Cu) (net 23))
 (segment (start 138.938 123.698) (end 138.938 123.19) (width 0.508) (layer F.Cu) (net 23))
 (segment (start 138.938 123.19) (end 139.065 123.063) (width 0.508) (layer F.Cu) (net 23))
 (segment (start 139.065 123.063) (end 139.065 95.758) (width 0.508) (layer F.Cu) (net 23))
 (via (at 143.383 95.504) (size 0.762) (layers F.Cu B.Cu) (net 23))
 (via (at 139.065 95.758) (size 0.762) (layers F.Cu B.Cu) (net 23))
 (segment (start 144.399 98.171) (end 154.178 107.95) (width 0.508) (layer F.Cu) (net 24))
 (segment (start 154.178 107.95) (end 154.178 114.046) (width 0.508) (layer F.Cu) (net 24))
 (segment (start 154.178 114.046) (end 154.305 114.173) (width 0.508) (layer F.Cu) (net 24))
 (segment (start 154.305 114.173) (end 154.305 114.427) (width 0.508) (layer F.Cu) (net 24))
 (segment (start 154.305 114.427) (end 154.432 114.554) (width 0.508) (layer F.Cu) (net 24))
 (segment (start 154.432 114.554) (end 154.432 114.681) (width 0.508) (layer F.Cu) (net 24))
 (segment (start 154.432 114.681) (end 154.559 114.808) (width 0.508) (layer F.Cu) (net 24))
 (segment (start 154.559 114.808) (end 154.559 115.062) (width 0.508) (layer F.Cu) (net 24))
 (segment (start 154.559 115.062) (end 154.813 115.316) (width 0.508) (layer F.Cu) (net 24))
 (segment (start 154.813 115.316) (end 154.813 115.443) (width 0.508) (layer F.Cu) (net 24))
 (segment (start 154.813 115.443) (end 155.067 115.697) (width 0.508) (layer F.Cu) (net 24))
 (segment (start 155.067 115.697) (end 155.067 116.459) (width 0.508) (layer F.Cu) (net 24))
 (segment (start 155.067 116.459) (end 155.194 116.586) (width 0.508) (layer F.Cu) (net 24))
 (segment (start 155.194 116.586) (end 155.194 116.84) (width 0.508) (layer F.Cu) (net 24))
 (segment (start 155.194 116.84) (end 155.448 117.094) (width 0.508) (layer F.Cu) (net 24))
 (segment (start 155.448 117.094) (end 155.448 117.221) (width 0.508) (layer F.Cu) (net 24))
 (segment (start 155.448 117.221) (end 156.591 118.364) (width 0.508) (layer F.Cu) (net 24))
 (segment (start 156.591 118.364) (end 156.591 118.618) (width 0.508) (layer F.Cu) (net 24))
 (segment (start 137.795 95.504) (end 139.954 93.345) (width 0.508) (layer B.Cu) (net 24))
 (segment (start 139.954 93.345) (end 141.859 93.345) (width 0.508) (layer B.Cu) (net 24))
 (segment (start 141.859 93.345) (end 141.986 93.472) (width 0.508) (layer B.Cu) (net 24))
 (segment (start 141.986 93.472) (end 142.24 93.472) (width 0.508) (layer B.Cu) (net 24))
 (segment (start 142.24 93.472) (end 142.367 93.599) (width 0.508) (layer B.Cu) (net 24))
 (segment (start 142.367 93.599) (end 142.494 93.599) (width 0.508) (layer B.Cu) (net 24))
 (segment (start 142.494 93.599) (end 142.621 93.726) (width 0.508) (layer B.Cu) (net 24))
 (segment (start 142.621 93.726) (end 142.875 93.726) (width 0.508) (layer B.Cu) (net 24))
 (segment (start 142.875 93.726) (end 143.129 93.98) (width 0.508) (layer B.Cu) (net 24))
 (segment (start 143.129 93.98) (end 143.256 93.98) (width 0.508) (layer B.Cu) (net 24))
 (segment (start 143.256 93.98) (end 143.891 94.615) (width 0.508) (layer B.Cu) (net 24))
 (segment (start 143.891 94.615) (end 144.018 94.615) (width 0.508) (layer B.Cu) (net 24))
 (segment (start 144.018 94.615) (end 144.272 94.869) (width 0.508) (layer B.Cu) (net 24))
 (segment (start 144.272 94.869) (end 144.272 94.996) (width 0.508) (layer B.Cu) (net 24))
 (segment (start 144.272 94.996) (end 144.399 95.123) (width 0.508) (layer B.Cu) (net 24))
 (segment (start 144.399 95.123) (end 144.399 98.171) (width 0.508) (layer B.Cu) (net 24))
 (segment (start 134.493 120.65) (end 137.795 117.348) (width 0.508) (layer F.Cu) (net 24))
 (segment (start 137.795 117.348) (end 137.795 95.504) (width 0.508) (layer F.Cu) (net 24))
 (segment (start 123.19 131.953) (end 134.493 120.65) (width 0.508) (layer B.Cu) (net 24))
 (segment (start 115.57 139.573) (end 123.19 131.953) (width 0.508) (layer F.Cu) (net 24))
 (via (at 144.399 98.171) (size 0.762) (layers F.Cu B.Cu) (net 24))
 (via (at 137.795 95.504) (size 0.762) (layers F.Cu B.Cu) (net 24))
 (via (at 134.493 120.65) (size 0.762) (layers F.Cu B.Cu) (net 24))
 (via (at 123.19 131.953) (size 0.762) (layers F.Cu B.Cu) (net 24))
 (segment (start 157.48 139.954) (end 159.004 138.43) (width 0.508) (layer F.Cu) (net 26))
 (segment (start 159.004 138.43) (end 159.004 123.19) (width 0.508) (layer F.Cu) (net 26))
 (segment (start 159.004 123.19) (end 158.877 123.063) (width 0.508) (layer F.Cu) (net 26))
 (segment (start 158.877 123.063) (end 158.877 122.809) (width 0.508) (layer F.Cu) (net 26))
 (segment (start 158.877 122.809) (end 158.75 122.682) (width 0.508) (layer F.Cu) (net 26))
 (segment (start 158.75 122.682) (end 158.75 122.555) (width 0.508) (layer F.Cu) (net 26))
 (segment (start 158.75 122.555) (end 158.623 122.428) (width 0.508) (layer F.Cu) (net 26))
 (segment (start 158.623 122.428) (end 158.623 122.174) (width 0.508) (layer F.Cu) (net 26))
 (segment (start 158.623 122.174) (end 158.369 121.92) (width 0.508) (layer F.Cu) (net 26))
 (segment (start 158.369 121.92) (end 158.369 121.793) (width 0.508) (layer F.Cu) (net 26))
 (segment (start 158.369 121.793) (end 158.115 121.539) (width 0.508) (layer F.Cu) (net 26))
 (segment (start 158.115 121.539) (end 158.115 108.077) (width 0.508) (layer F.Cu) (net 26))
 (segment (start 158.115 108.077) (end 157.988 107.95) (width 0.508) (layer F.Cu) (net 26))
 (segment (start 157.988 107.95) (end 157.988 107.696) (width 0.508) (layer F.Cu) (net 26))
 (segment (start 157.988 107.696) (end 157.734 107.442) (width 0.508) (layer F.Cu) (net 26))
 (segment (start 157.734 107.442) (end 157.734 107.315) (width 0.508) (layer F.Cu) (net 26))
 (segment (start 157.734 107.315) (end 156.591 106.172) (width 0.508) (layer F.Cu) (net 26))
 (segment (start 156.591 106.172) (end 156.591 105.918) (width 0.508) (layer F.Cu) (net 26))
 (segment (start 147.955 137.668) (end 144.526 137.668) (width 0.508) (layer F.Cu) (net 30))
 (segment (start 144.526 137.668) (end 142.367 139.827) (width 0.508) (layer F.Cu) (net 30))
 (segment (start 171.704 127.762) (end 161.798 137.668) (width 0.508) (layer B.Cu) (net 30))
 (segment (start 161.798 137.668) (end 147.955 137.668) (width 0.508) (layer B.Cu) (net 30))
 (segment (start 171.577 107.569) (end 171.704 107.696) (width 0.508) (layer F.Cu) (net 30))
 (segment (start 171.704 107.696) (end 171.704 127.762) (width 0.508) (layer F.Cu) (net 30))
 (segment (start 163.83 106.553) (end 170.561 106.553) (width 0.508) (layer B.Cu) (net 30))
 (segment (start 170.561 106.553) (end 171.577 107.569) (width 0.508) (layer B.Cu) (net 30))
 (segment (start 162.179 108.204) (end 163.83 106.553) (width 0.508) (layer F.Cu) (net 30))
 (segment (start 156.591 113.538) (end 161.925 108.204) (width 0.508) (layer B.Cu) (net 30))
 (segment (start 161.925 108.204) (end 162.179 108.204) (width 0.508) (layer B.Cu) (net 30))
 (via (at 147.955 137.668) (size 0.762) (layers F.Cu B.Cu) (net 30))
 (via (at 171.704 127.762) (size 0.762) (layers F.Cu B.Cu) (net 30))
 (via (at 171.577 107.569) (size 0.762) (layers F.Cu B.Cu) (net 30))
 (via (at 163.83 106.553) (size 0.762) (layers F.Cu B.Cu) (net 30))
 (via (at 162.179 108.204) (size 0.762) (layers F.Cu B.Cu) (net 30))
 (segment (start 160.528 103.378) (end 156.591 103.378) (width 0.508) (layer B.Cu) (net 31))
 (segment (start 165.227 99.695) (end 164.211 99.695) (width 0.508) (layer F.Cu) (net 31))
 (segment (start 164.211 99.695) (end 160.528 103.378) (width 0.508) (layer F.Cu) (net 31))
 (via (at 160.528 103.378) (size 0.762) (layers F.Cu B.Cu) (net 31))
 (segment (start 164.973 122.428) (end 163.703 123.698) (width 0.508) (layer B.Cu) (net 33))
 (segment (start 163.703 123.698) (end 156.591 123.698) (width 0.508) (layer B.Cu) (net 33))
 (segment (start 160.147 134.493) (end 167.259 127.381) (width 0.508) (layer F.Cu) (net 33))
 (segment (start 167.259 127.381) (end 167.259 122.428) (width 0.508) (layer F.Cu) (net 33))
 (segment (start 167.259 122.428) (end 167.132 122.301) (width 0.508) (layer F.Cu) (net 33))
 (segment (start 167.132 122.301) (end 167.132 122.174) (width 0.508) (layer F.Cu) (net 33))
 (segment (start 167.132 122.174) (end 166.878 121.92) (width 0.508) (layer F.Cu) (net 33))
 (segment (start 166.878 121.92) (end 166.751 121.92) (width 0.508) (layer F.Cu) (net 33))
 (segment (start 166.751 121.92) (end 166.624 121.793) (width 0.508) (layer F.Cu) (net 33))
 (segment (start 166.624 121.793) (end 165.608 121.793) (width 0.508) (layer F.Cu) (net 33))
 (segment (start 165.608 121.793) (end 164.973 122.428) (width 0.508) (layer F.Cu) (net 33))
 (segment (start 119.38 129.794) (end 125.095 135.509) (width 0.508) (layer B.Cu) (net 33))
 (segment (start 125.095 135.509) (end 155.448 135.509) (width 0.508) (layer B.Cu) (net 33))
 (segment (start 155.448 135.509) (end 155.575 135.382) (width 0.508) (layer B.Cu) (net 33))
 (segment (start 155.575 135.382) (end 155.702 135.382) (width 0.508) (layer B.Cu) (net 33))
 (segment (start 155.702 135.382) (end 156.591 134.493) (width 0.508) (layer B.Cu) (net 33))
 (segment (start 156.591 134.493) (end 160.147 134.493) (width 0.508) (layer B.Cu) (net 33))
 (segment (start 115.062 125.476) (end 119.38 129.794) (width 0.508) (layer F.Cu) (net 33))
 (via (at 164.973 122.428) (size 0.762) (layers F.Cu B.Cu) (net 33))
 (via (at 160.147 134.493) (size 0.762) (layers F.Cu B.Cu) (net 33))
 (via (at 119.38 129.794) (size 0.762) (layers F.Cu B.Cu) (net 33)))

